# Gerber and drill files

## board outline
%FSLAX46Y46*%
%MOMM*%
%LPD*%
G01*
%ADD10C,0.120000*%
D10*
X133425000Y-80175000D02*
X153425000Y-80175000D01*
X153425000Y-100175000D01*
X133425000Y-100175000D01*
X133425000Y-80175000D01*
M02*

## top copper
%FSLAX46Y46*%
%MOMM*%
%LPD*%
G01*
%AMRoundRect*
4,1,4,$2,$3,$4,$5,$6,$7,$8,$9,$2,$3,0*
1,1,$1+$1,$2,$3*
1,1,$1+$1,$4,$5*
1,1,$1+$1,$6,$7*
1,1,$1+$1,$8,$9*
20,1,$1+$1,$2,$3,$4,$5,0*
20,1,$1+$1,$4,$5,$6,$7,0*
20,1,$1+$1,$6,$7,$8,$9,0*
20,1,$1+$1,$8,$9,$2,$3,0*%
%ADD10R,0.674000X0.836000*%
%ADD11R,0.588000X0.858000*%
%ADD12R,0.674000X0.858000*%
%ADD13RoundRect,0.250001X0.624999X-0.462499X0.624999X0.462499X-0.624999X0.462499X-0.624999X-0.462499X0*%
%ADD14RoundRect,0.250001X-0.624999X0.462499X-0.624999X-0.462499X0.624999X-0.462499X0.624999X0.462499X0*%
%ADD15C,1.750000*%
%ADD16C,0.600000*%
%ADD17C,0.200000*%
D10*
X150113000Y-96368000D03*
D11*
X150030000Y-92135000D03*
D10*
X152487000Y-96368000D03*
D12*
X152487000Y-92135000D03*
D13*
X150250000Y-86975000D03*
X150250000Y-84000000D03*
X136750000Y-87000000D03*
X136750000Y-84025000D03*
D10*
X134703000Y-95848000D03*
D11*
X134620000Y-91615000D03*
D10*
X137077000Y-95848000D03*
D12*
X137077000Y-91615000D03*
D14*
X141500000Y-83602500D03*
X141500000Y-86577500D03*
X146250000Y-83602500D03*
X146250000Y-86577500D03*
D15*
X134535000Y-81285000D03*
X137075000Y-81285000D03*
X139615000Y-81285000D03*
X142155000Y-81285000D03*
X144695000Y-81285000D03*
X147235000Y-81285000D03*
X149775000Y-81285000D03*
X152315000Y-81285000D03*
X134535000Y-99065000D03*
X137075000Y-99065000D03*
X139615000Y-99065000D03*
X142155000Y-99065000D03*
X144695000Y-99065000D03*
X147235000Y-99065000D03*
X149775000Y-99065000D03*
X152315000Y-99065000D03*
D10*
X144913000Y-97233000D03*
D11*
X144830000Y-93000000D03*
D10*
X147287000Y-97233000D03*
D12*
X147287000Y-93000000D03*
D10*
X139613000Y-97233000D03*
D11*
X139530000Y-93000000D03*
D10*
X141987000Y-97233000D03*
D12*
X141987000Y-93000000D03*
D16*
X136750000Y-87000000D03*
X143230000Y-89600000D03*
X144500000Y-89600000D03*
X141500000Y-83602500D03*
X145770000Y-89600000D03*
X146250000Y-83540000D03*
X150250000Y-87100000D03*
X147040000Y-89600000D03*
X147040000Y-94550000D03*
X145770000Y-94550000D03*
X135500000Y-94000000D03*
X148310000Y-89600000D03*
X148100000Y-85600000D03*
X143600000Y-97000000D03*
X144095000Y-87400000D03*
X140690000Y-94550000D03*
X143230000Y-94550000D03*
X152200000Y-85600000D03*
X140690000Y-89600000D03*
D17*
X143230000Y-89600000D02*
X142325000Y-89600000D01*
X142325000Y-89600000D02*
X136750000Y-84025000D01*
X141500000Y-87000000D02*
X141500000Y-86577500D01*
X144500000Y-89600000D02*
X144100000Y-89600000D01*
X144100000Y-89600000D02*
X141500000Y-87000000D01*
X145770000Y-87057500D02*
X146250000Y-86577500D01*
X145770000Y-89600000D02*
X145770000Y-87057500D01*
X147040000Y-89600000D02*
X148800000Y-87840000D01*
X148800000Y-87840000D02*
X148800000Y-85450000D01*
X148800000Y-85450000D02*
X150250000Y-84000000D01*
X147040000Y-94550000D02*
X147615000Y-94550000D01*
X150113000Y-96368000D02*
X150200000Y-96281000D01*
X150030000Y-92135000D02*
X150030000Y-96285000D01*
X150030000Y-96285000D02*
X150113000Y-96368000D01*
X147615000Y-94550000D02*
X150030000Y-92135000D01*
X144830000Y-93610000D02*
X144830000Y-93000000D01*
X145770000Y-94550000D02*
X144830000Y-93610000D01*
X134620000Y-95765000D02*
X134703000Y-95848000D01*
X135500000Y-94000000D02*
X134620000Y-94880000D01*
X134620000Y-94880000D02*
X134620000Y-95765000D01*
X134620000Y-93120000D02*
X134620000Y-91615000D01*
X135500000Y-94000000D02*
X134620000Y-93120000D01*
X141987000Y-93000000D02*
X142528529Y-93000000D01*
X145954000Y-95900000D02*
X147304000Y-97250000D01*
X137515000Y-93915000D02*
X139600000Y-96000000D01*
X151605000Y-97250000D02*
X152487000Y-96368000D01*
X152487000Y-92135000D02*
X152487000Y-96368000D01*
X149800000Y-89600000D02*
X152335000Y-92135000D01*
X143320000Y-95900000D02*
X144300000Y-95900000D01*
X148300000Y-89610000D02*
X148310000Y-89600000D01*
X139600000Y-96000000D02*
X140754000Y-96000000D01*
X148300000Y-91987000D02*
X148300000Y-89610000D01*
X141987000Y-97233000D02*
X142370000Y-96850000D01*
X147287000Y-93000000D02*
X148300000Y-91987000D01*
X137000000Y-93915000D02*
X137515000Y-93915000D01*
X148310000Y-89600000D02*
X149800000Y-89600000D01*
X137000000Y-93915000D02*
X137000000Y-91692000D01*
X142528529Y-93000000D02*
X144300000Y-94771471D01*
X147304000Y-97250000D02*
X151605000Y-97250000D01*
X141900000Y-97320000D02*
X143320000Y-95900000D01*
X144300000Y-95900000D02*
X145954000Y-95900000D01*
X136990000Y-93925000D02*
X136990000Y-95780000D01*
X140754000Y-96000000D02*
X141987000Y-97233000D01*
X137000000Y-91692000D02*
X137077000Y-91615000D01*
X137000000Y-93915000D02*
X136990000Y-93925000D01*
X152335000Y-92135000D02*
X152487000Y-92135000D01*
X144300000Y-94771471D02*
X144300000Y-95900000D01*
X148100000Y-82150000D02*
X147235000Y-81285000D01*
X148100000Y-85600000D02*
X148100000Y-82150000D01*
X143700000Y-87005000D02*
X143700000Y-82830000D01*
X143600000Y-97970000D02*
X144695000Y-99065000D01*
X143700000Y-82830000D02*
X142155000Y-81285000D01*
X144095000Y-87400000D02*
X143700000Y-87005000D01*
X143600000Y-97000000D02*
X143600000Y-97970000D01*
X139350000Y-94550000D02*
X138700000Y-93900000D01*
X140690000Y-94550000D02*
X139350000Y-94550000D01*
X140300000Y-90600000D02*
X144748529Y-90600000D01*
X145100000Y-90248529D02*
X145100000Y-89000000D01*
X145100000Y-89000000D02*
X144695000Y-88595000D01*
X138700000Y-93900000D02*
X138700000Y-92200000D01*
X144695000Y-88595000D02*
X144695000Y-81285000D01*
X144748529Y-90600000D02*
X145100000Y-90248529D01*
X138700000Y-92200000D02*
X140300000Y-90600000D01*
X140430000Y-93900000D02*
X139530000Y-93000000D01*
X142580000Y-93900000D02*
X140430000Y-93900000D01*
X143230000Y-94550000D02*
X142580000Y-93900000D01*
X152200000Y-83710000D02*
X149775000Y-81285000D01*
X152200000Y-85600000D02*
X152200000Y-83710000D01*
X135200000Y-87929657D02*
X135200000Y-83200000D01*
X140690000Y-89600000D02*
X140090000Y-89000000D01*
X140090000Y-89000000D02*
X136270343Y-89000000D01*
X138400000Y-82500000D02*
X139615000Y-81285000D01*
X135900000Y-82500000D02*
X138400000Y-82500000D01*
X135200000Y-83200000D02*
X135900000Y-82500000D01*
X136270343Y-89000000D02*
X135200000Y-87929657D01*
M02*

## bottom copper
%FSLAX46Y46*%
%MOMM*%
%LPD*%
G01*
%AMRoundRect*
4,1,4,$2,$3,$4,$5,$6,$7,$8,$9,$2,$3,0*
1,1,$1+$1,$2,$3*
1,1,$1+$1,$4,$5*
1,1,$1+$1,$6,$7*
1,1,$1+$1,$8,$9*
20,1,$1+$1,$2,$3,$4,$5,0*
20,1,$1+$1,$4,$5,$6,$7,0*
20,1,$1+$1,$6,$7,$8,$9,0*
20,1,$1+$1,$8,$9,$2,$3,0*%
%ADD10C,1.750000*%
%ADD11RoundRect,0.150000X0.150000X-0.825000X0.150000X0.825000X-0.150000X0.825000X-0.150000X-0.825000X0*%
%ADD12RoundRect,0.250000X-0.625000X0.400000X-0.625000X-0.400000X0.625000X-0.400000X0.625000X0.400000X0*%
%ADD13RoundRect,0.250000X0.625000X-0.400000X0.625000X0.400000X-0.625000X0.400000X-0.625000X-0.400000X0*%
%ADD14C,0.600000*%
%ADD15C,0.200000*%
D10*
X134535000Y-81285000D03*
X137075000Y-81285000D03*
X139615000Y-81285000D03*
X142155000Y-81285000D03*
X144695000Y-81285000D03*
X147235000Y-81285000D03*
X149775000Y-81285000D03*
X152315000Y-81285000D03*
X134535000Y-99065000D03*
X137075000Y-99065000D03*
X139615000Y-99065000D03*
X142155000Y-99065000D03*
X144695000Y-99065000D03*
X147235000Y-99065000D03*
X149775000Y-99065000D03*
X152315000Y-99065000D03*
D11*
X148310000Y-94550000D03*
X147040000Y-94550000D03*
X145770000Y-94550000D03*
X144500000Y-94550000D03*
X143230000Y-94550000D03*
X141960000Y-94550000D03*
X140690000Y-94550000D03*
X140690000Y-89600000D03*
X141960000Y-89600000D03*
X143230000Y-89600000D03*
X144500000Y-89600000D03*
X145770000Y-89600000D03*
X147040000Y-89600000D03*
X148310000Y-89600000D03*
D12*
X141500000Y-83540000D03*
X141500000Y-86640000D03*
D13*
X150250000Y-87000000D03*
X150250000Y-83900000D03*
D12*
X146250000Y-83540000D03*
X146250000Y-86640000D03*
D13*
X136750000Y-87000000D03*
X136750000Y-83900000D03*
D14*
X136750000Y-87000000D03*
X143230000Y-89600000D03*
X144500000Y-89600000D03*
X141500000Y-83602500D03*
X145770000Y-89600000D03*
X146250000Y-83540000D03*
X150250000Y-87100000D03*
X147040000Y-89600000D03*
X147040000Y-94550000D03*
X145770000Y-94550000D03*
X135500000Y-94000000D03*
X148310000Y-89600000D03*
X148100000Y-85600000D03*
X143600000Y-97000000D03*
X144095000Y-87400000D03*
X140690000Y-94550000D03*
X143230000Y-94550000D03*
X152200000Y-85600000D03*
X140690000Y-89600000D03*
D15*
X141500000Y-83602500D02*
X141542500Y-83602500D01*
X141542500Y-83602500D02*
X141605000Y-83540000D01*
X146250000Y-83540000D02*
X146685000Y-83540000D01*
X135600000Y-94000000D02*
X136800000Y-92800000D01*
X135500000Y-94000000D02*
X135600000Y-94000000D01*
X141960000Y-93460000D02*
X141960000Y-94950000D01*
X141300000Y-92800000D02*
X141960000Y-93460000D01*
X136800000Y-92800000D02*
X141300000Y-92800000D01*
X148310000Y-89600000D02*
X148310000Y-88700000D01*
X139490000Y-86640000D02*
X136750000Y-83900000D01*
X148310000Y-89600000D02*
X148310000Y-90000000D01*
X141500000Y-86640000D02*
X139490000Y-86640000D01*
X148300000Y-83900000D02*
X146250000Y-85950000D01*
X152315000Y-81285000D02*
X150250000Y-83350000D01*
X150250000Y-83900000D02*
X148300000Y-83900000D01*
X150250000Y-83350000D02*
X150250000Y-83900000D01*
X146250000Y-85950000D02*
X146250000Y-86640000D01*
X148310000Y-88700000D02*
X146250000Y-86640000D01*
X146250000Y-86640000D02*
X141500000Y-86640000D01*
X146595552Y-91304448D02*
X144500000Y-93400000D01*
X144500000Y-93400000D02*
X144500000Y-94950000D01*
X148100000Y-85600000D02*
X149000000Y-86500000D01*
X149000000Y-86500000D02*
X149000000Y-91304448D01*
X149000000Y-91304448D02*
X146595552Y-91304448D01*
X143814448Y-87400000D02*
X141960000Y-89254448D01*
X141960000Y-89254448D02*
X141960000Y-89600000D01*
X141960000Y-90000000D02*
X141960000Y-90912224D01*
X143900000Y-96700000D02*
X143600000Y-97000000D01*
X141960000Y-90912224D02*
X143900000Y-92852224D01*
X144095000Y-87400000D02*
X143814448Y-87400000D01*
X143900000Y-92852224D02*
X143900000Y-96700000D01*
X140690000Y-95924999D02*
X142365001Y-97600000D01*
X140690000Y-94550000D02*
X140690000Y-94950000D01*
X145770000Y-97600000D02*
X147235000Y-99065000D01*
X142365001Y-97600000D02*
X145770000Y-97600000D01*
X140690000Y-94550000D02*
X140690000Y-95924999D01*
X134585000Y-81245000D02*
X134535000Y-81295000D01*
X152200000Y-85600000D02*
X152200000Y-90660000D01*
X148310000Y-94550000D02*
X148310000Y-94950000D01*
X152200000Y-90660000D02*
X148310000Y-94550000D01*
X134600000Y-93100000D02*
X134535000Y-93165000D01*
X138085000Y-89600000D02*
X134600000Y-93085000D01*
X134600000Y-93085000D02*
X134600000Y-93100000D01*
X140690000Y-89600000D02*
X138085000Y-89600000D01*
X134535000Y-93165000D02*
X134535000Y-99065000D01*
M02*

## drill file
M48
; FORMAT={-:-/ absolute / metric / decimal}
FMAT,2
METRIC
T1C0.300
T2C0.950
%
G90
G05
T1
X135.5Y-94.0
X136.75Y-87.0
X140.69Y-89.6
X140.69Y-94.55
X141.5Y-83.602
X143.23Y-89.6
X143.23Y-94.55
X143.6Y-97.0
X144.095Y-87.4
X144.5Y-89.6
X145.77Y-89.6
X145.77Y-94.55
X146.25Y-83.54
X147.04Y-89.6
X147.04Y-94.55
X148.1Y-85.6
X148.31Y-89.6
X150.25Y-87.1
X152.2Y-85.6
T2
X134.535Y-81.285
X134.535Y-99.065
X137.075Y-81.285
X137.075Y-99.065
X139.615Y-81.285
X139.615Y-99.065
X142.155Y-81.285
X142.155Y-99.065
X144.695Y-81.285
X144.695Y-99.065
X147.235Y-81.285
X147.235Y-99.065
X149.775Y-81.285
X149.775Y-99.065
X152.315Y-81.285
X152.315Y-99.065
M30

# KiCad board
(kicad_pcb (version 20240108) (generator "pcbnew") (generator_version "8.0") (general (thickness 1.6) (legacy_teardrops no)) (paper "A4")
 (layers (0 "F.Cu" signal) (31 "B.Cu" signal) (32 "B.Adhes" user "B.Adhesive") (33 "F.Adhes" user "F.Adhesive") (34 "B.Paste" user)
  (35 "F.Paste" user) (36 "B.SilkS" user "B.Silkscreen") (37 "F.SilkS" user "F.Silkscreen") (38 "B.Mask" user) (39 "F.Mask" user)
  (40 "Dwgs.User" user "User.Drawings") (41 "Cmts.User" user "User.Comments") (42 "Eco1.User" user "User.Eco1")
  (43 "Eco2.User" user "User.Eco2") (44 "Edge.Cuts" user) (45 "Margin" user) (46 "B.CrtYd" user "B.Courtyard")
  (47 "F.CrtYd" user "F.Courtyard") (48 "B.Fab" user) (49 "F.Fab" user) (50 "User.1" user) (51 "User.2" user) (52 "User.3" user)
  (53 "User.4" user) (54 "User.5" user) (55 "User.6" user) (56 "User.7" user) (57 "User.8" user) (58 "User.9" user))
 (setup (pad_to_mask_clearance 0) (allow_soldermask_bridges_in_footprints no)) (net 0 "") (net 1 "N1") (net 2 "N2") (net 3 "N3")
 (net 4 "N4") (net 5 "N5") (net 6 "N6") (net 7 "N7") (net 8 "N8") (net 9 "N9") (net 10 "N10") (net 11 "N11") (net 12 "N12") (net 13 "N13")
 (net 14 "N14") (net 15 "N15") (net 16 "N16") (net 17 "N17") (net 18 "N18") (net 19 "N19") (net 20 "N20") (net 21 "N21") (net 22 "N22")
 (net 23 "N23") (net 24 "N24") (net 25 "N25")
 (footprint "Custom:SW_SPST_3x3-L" (layer "F.Cu") (at 151.3 94.5 90)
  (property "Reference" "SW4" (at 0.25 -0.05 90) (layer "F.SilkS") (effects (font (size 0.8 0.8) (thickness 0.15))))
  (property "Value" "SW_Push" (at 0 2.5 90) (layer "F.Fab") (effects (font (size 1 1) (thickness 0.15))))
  (pad "1" smd rect (at -1.868 -1.187 90) (size 0.836 0.674) (layers "F.Cu" "F.Paste" "F.Mask") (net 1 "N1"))
  (pad "1" smd rect (at 2.365 -1.27 90) (size 0.858 0.588) (layers "F.Cu" "F.Paste" "F.Mask") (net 1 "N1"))
  (pad "2" smd rect (at -1.868 1.187 90) (size 0.836 0.674) (layers "F.Cu" "F.Paste" "F.Mask") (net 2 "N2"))
  (pad "2" smd rect (at 2.365 1.187 90) (size 0.858 0.674) (layers "F.Cu" "F.Paste" "F.Mask") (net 2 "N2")))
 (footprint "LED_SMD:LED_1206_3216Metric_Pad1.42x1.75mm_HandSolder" (layer "F.Cu") (at 150.25 85.4875 90)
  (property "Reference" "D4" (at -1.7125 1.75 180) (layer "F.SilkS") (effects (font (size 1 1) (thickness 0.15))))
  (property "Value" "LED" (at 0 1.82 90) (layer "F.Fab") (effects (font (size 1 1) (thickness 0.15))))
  (pad "1" smd roundrect (at -1.4875 0 90) (size 1.425 1.75) (layers "F.Cu" "F.Paste" "F.Mask") (roundrect_rratio 0.175439) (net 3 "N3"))
  (pad "2" smd roundrect (at 1.4875 0 90) (size 1.425 1.75) (layers "F.Cu" "F.Paste" "F.Mask") (roundrect_rratio 0.175439) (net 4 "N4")))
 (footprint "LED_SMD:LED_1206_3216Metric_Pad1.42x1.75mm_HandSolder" (layer "F.Cu") (at 136.75 85.5125 90)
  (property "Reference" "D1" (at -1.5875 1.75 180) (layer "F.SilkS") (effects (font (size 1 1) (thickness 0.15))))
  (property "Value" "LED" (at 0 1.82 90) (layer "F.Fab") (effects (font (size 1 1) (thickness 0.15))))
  (pad "1" smd roundrect (at -1.4875 0 90) (size 1.425 1.75) (layers "F.Cu" "F.Paste" "F.Mask") (roundrect_rratio 0.175439) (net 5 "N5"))
  (pad "2" smd roundrect (at 1.4875 0 90) (size 1.425 1.75) (layers "F.Cu" "F.Paste" "F.Mask") (roundrect_rratio 0.175439) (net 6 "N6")))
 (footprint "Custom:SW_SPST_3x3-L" (layer "F.Cu") (at 135.89 93.98 90)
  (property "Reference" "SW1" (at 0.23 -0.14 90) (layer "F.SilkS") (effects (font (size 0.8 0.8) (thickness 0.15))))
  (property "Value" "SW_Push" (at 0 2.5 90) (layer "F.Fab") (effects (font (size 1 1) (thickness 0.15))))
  (pad "1" smd rect (at -1.868 -1.187 90) (size 0.836 0.674) (layers "F.Cu" "F.Paste" "F.Mask") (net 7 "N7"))
  (pad "1" smd rect (at 2.365 -1.27 90) (size 0.858 0.588) (layers "F.Cu" "F.Paste" "F.Mask") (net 7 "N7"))
  (pad "2" smd rect (at -1.868 1.187 90) (size 0.836 0.674) (layers "F.Cu" "F.Paste" "F.Mask") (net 2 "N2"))
  (pad "2" smd rect (at 2.365 1.187 90) (size 0.858 0.674) (layers "F.Cu" "F.Paste" "F.Mask") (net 2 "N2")))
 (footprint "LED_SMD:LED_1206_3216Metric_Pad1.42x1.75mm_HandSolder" (layer "F.Cu") (at 141.5 85.09 -90)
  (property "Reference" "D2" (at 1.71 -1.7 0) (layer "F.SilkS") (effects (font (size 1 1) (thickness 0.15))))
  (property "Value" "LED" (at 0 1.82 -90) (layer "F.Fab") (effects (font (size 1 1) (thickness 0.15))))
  (pad "1" smd roundrect (at -1.4875 0 270) (size 1.425 1.75) (layers "F.Cu" "F.Paste" "F.Mask") (roundrect_rratio 0.175439) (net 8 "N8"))
  (pad "2" smd roundrect (at 1.4875 0 270) (size 1.425 1.75) (layers "F.Cu" "F.Paste" "F.Mask") (roundrect_rratio 0.175439) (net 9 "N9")))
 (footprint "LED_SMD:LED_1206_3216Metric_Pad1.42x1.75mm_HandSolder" (layer "F.Cu") (at 146.25 85.09 -90)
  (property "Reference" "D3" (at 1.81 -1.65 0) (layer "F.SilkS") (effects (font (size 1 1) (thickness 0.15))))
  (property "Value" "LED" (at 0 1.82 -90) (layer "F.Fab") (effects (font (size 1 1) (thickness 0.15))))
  (pad "1" smd roundrect (at -1.4875 0 270) (size 1.425 1.75) (layers "F.Cu" "F.Paste" "F.Mask") (roundrect_rratio 0.175439) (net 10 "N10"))
  (pad "2" smd roundrect (at 1.4875 0 270) (size 1.425 1.75) (layers "F.Cu" "F.Paste" "F.Mask") (roundrect_rratio 0.175439) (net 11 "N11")))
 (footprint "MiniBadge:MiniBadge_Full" (layer "F.Cu") (at 133.265 80.015)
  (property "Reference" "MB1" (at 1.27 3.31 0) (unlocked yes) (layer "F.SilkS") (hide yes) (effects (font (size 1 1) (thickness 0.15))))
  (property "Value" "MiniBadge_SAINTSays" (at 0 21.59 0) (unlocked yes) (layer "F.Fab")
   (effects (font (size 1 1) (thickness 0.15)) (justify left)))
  (fp_rect (start 20.16 20.16) (end 0.16 0.16) (stroke (width 0.12) (type solid)) (fill none) (layer "Edge.Cuts"))
  (pad "1" thru_hole circle (at 1.27 1.27) (size 1.75 1.75) (drill 0.95) (layers "*.Cu" "*.Mask") (remove_unused_layers no) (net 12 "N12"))
  (pad "2" thru_hole circle (at 3.81 1.27) (size 1.75 1.75) (drill 0.95) (layers "*.Cu" "*.Mask") (remove_unused_layers no) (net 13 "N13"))
  (pad "3" thru_hole circle (at 6.35 1.27 90) (size 1.75 1.75) (drill 0.95) (layers "*.Cu" "*.Mask") (remove_unused_layers no)
   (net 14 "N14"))
  (pad "4" thru_hole circle (at 8.89 1.27) (size 1.75 1.75) (drill 0.95) (layers "*.Cu" "*.Mask") (remove_unused_layers no) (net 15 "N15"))
  (pad "5" thru_hole circle (at 11.43 1.27) (size 1.75 1.75) (drill 0.95) (layers "*.Cu" "*.Mask") (remove_unused_layers no) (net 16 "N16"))
  (pad "6" thru_hole circle (at 13.97 1.27) (size 1.75 1.75) (drill 0.95) (layers "*.Cu" "*.Mask") (remove_unused_layers no) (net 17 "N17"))
  (pad "7" thru_hole circle (at 16.51 1.27) (size 1.75 1.75) (drill 0.95) (layers "*.Cu" "*.Mask") (remove_unused_layers no) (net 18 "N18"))
  (pad "8" thru_hole circle (at 19.05 1.27) (size 1.75 1.75) (drill 0.95) (layers "*.Cu" "*.Mask") (remove_unused_layers no) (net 2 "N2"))
  (pad "9" thru_hole circle (at 1.27 19.05) (size 1.75 1.75) (drill 0.95) (layers "*.Cu" "*.Mask") (remove_unused_layers no) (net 14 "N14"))
  (pad "10" thru_hole circle (at 3.81 19.05) (size 1.75 1.75) (drill 0.95) (layers "*.Cu" "*.Mask") (remove_unused_layers no) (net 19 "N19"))
  (pad "11" thru_hole circle (at 6.35 19.05) (size 1.75 1.75) (drill 0.95) (layers "*.Cu" "*.Mask") (remove_unused_layers no) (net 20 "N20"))
  (pad "12" thru_hole circle (at 8.89 19.05) (size 1.75 1.75) (drill 0.95) (layers "*.Cu" "*.Mask") (remove_unused_layers no) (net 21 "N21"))
  (pad "13" thru_hole circle (at 11.43 19.05) (size 1.75 1.75) (drill 0.95) (layers "*.Cu" "*.Mask") (remove_unused_layers no)
   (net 15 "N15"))
  (pad "14" thru_hole circle (at 13.97 19.05) (size 1.75 1.75) (drill 0.95) (layers "*.Cu" "*.Mask") (remove_unused_layers no)
   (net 16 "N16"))
  (pad "15" thru_hole circle (at 16.51 19.05) (size 1.75 1.75) (drill 0.95) (layers "*.Cu" "*.Mask") (remove_unused_layers no)
   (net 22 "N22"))
  (pad "16" thru_hole circle (at 19.05 19.05) (size 1.75 1.75) (drill 0.95) (layers "*.Cu" "*.Mask") (remove_unused_layers no)
   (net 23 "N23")))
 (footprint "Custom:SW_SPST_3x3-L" (layer "F.Cu") (at 146.1 95.365 90)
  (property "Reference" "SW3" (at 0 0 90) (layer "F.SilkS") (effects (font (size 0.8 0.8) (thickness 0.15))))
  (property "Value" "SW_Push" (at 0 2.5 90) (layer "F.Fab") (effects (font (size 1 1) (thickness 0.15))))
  (pad "1" smd rect (at -1.868 -1.187 90) (size 0.836 0.674) (layers "F.Cu" "F.Paste" "F.Mask") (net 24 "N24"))
  (pad "1" smd rect (at 2.365 -1.27 90) (size 0.858 0.588) (layers "F.Cu" "F.Paste" "F.Mask") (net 24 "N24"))
  (pad "2" smd rect (at -1.868 1.187 90) (size 0.836 0.674) (layers "F.Cu" "F.Paste" "F.Mask") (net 2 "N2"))
  (pad "2" smd rect (at 2.365 1.187 90) (size 0.858 0.674) (layers "F.Cu" "F.Paste" "F.Mask") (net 2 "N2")))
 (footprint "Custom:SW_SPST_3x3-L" (layer "F.Cu") (at 140.8 95.365 90)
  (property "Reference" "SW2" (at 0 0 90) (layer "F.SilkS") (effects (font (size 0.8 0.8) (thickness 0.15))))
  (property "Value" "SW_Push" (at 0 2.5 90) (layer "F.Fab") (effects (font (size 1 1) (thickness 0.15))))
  (pad "1" smd rect (at -1.868 -1.187 90) (size 0.836 0.674) (layers "F.Cu" "F.Paste" "F.Mask") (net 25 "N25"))
  (pad "1" smd rect (at 2.365 -1.27 90) (size 0.858 0.588) (layers "F.Cu" "F.Paste" "F.Mask") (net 25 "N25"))
  (pad "2" smd rect (at -1.868 1.187 90) (size 0.836 0.674) (layers "F.Cu" "F.Paste" "F.Mask") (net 2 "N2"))
  (pad "2" smd rect (at 2.365 1.187 90) (size 0.858 0.674) (layers "F.Cu" "F.Paste" "F.Mask") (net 2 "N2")))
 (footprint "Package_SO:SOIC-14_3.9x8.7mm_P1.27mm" (layer "B.Cu") (at 144.5 92.075 90)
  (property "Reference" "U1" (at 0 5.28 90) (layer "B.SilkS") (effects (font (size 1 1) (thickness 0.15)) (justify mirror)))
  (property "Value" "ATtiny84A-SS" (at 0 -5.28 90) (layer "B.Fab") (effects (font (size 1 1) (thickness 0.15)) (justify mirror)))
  (pad "1" smd roundrect (at -2.475 3.81 90) (size 1.95 0.6) (layers "B.Cu" "B.Paste" "B.Mask") (roundrect_rratio 0.25) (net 18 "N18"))
  (pad "2" smd roundrect (at -2.475 2.54 90) (size 1.95 0.6) (layers "B.Cu" "B.Paste" "B.Mask") (roundrect_rratio 0.25) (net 1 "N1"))
  (pad "3" smd roundrect (at -2.475 1.27 90) (size 1.95 0.6) (layers "B.Cu" "B.Paste" "B.Mask") (roundrect_rratio 0.25) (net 24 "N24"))
  (pad "4" smd roundrect (at -2.475 0 90) (size 1.95 0.6) (layers "B.Cu" "B.Paste" "B.Mask") (roundrect_rratio 0.25) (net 17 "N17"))
  (pad "5" smd roundrect (at -2.475 -1.27 90) (size 1.95 0.6) (layers "B.Cu" "B.Paste" "B.Mask") (roundrect_rratio 0.25) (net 25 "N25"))
  (pad "6" smd roundrect (at -2.475 -2.54 90) (size 1.95 0.6) (layers "B.Cu" "B.Paste" "B.Mask") (roundrect_rratio 0.25) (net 7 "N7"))
  (pad "7" smd roundrect (at -2.475 -3.81 90) (size 1.95 0.6) (layers "B.Cu" "B.Paste" "B.Mask") (roundrect_rratio 0.25) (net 16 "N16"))
  (pad "8" smd roundrect (at 2.475 -3.81 90) (size 1.95 0.6) (layers "B.Cu" "B.Paste" "B.Mask") (roundrect_rratio 0.25) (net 14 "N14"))
  (pad "9" smd roundrect (at 2.475 -2.54 90) (size 1.95 0.6) (layers "B.Cu" "B.Paste" "B.Mask") (roundrect_rratio 0.25) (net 15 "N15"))
  (pad "10" smd roundrect (at 2.475 -1.27 90) (size 1.95 0.6) (layers "B.Cu" "B.Paste" "B.Mask") (roundrect_rratio 0.25) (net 6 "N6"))
  (pad "11" smd roundrect (at 2.475 0 90) (size 1.95 0.6) (layers "B.Cu" "B.Paste" "B.Mask") (roundrect_rratio 0.25) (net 9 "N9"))
  (pad "12" smd roundrect (at 2.475 1.27 90) (size 1.95 0.6) (layers "B.Cu" "B.Paste" "B.Mask") (roundrect_rratio 0.25) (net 11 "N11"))
  (pad "13" smd roundrect (at 2.475 2.54 90) (size 1.95 0.6) (layers "B.Cu" "B.Paste" "B.Mask") (roundrect_rratio 0.25) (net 4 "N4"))
  (pad "14" smd roundrect (at 2.475 3.81 90) (size 1.95 0.6) (layers "B.Cu" "B.Paste" "B.Mask") (roundrect_rratio 0.25) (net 2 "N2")))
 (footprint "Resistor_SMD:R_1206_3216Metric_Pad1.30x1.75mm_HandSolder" (layer "B.Cu") (at 141.5 85.09 -90)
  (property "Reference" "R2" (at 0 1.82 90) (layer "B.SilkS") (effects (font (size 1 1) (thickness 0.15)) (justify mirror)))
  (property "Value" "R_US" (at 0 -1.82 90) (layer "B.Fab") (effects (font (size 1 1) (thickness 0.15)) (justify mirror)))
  (pad "1" smd roundrect (at -1.55 0 270) (size 1.3 1.75) (layers "B.Cu" "B.Paste" "B.Mask") (roundrect_rratio 0.192308) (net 8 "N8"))
  (pad "2" smd roundrect (at 1.55 0 270) (size 1.3 1.75) (layers "B.Cu" "B.Paste" "B.Mask") (roundrect_rratio 0.192308) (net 2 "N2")))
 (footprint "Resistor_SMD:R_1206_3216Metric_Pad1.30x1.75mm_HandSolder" (layer "B.Cu") (at 150.25 85.45 90)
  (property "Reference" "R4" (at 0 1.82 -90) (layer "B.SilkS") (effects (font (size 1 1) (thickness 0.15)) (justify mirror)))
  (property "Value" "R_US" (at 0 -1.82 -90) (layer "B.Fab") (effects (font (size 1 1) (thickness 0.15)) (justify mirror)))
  (pad "1" smd roundrect (at -1.55 0 90) (size 1.3 1.75) (layers "B.Cu" "B.Paste" "B.Mask") (roundrect_rratio 0.192308) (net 3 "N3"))
  (pad "2" smd roundrect (at 1.55 0 90) (size 1.3 1.75) (layers "B.Cu" "B.Paste" "B.Mask") (roundrect_rratio 0.192308) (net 2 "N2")))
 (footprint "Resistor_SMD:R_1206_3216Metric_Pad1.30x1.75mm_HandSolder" (layer "B.Cu") (at 146.25 85.09 -90)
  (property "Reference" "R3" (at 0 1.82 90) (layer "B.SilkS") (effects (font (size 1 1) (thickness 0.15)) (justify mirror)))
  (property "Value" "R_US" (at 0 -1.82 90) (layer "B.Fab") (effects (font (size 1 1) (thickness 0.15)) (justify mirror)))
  (pad "1" smd roundrect (at -1.55 0 270) (size 1.3 1.75) (layers "B.Cu" "B.Paste" "B.Mask") (roundrect_rratio 0.192308) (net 10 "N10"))
  (pad "2" smd roundrect (at 1.55 0 270) (size 1.3 1.75) (layers "B.Cu" "B.Paste" "B.Mask") (roundrect_rratio 0.192308) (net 2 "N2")))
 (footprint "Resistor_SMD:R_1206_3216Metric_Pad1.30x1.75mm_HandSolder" (layer "B.Cu") (at 136.75 85.45 90)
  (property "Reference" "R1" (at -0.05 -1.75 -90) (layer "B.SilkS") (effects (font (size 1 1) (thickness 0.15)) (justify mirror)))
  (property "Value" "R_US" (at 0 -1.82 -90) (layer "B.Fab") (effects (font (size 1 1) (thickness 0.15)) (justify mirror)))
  (pad "1" smd roundrect (at -1.55 0 90) (size 1.3 1.75) (layers "B.Cu" "B.Paste" "B.Mask") (roundrect_rratio 0.192308) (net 5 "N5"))
  (pad "2" smd roundrect (at 1.55 0 90) (size 1.3 1.75) (layers "B.Cu" "B.Paste" "B.Mask") (roundrect_rratio 0.192308) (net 2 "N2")))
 (via (at 136.75 87) (size 0.6) (drill 0.3) (layers "F.Cu" "B.Cu") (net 5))
 (segment (start 143.23 89.6) (end 142.325 89.6) (width 0.2) (layer "F.Cu") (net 6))
 (segment (start 142.325 89.6) (end 136.75 84.025) (width 0.2) (layer "F.Cu") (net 6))
 (via (at 143.23 89.6) (size 0.6) (drill 0.3) (layers "F.Cu" "B.Cu") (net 6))
 (segment (start 141.5 87) (end 141.5 86.5775) (width 0.2) (layer "F.Cu") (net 9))
 (segment (start 144.5 89.6) (end 144.1 89.6) (width 0.2) (layer "F.Cu") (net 9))
 (segment (start 144.1 89.6) (end 141.5 87) (width 0.2) (layer "F.Cu") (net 9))
 (via (at 144.5 89.6) (size 0.6) (drill 0.3) (layers "F.Cu" "B.Cu") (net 9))
 (via (at 141.5 83.6025) (size 0.6) (drill 0.3) (layers "F.Cu" "B.Cu") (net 8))
 (segment (start 141.5 83.6025) (end 141.5425 83.6025) (width 0.2) (layer "B.Cu") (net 8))
 (segment (start 141.5425 83.6025) (end 141.605 83.54) (width 0.2) (layer "B.Cu") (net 8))
 (segment (start 145.77 87.0575) (end 146.25 86.5775) (width 0.2) (layer "F.Cu") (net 11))
 (segment (start 145.77 89.6) (end 145.77 87.0575) (width 0.2) (layer "F.Cu") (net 11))
 (via (at 145.77 89.6) (size 0.6) (drill 0.3) (layers "F.Cu" "B.Cu") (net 11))
 (via (at 146.25 83.54) (size 0.6) (drill 0.3) (layers "F.Cu" "B.Cu") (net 10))
 (segment (start 146.25 83.54) (end 146.685 83.54) (width 0.2) (layer "B.Cu") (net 10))
 (via (at 150.25 87.1) (size 0.6) (drill 0.3) (layers "F.Cu" "B.Cu") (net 3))
 (segment (start 147.04 89.6) (end 148.8 87.84) (width 0.2) (layer "F.Cu") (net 4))
 (segment (start 148.8 87.84) (end 148.8 85.45) (width 0.2) (layer "F.Cu") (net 4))
 (segment (start 148.8 85.45) (end 150.25 84) (width 0.2) (layer "F.Cu") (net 4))
 (via (at 147.04 89.6) (size 0.6) (drill 0.3) (layers "F.Cu" "B.Cu") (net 4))
 (segment (start 147.04 94.55) (end 147.615 94.55) (width 0.2) (layer "F.Cu") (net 1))
 (segment (start 150.113 96.368) (end 150.2 96.281) (width 0.2) (layer "F.Cu") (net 1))
 (segment (start 150.03 92.135) (end 150.03 96.285) (width 0.2) (layer "F.Cu") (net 1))
 (segment (start 150.03 96.285) (end 150.113 96.368) (width 0.2) (layer "F.Cu") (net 1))
 (segment (start 147.615 94.55) (end 150.03 92.135) (width 0.2) (layer "F.Cu") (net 1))
 (via (at 147.04 94.55) (size 0.6) (drill 0.3) (layers "F.Cu" "B.Cu") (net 1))
 (segment (start 144.83 93.61) (end 144.83 93) (width 0.2) (layer "F.Cu") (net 24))
 (segment (start 145.77 94.55) (end 144.83 93.61) (width 0.2) (layer "F.Cu") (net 24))
 (via (at 145.77 94.55) (size 0.6) (drill 0.3) (layers "F.Cu" "B.Cu") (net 24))
 (segment (start 134.62 95.765) (end 134.703 95.848) (width 0.2) (layer "F.Cu") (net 7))
 (segment (start 135.5 94) (end 134.62 94.88) (width 0.2) (layer "F.Cu") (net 7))
 (segment (start 134.62 94.88) (end 134.62 95.765) (width 0.2) (layer "F.Cu") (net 7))
 (segment (start 134.62 93.12) (end 134.62 91.615) (width 0.2) (layer "F.Cu") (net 7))
 (segment (start 135.5 94) (end 134.62 93.12) (width 0.2) (layer "F.Cu") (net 7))
 (via (at 135.5 94) (size 0.6) (drill 0.3) (layers "F.Cu" "B.Cu") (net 7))
 (segment (start 135.6 94) (end 136.8 92.8) (width 0.2) (layer "B.Cu") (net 7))
 (segment (start 135.5 94) (end 135.6 94) (width 0.2) (layer "B.Cu") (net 7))
 (segment (start 141.96 93.46) (end 141.96 94.95) (width 0.2) (layer "B.Cu") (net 7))
 (segment (start 141.3 92.8) (end 141.96 93.46) (width 0.2) (layer "B.Cu") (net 7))
 (segment (start 136.8 92.8) (end 141.3 92.8) (width 0.2) (layer "B.Cu") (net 7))
 (segment (start 141.987 93) (end 142.528529 93) (width 0.2) (layer "F.Cu") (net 2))
 (segment (start 145.954 95.9) (end 147.304 97.25) (width 0.2) (layer "F.Cu") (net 2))
 (segment (start 137.515 93.915) (end 139.6 96) (width 0.2) (layer "F.Cu") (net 2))
 (segment (start 151.605 97.25) (end 152.487 96.368) (width 0.2) (layer "F.Cu") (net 2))
 (segment (start 152.487 92.135) (end 152.487 96.368) (width 0.2) (layer "F.Cu") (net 2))
 (segment (start 149.8 89.6) (end 152.335 92.135) (width 0.2) (layer "F.Cu") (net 2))
 (segment (start 143.32 95.9) (end 144.3 95.9) (width 0.2) (layer "F.Cu") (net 2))
 (segment (start 148.3 89.61) (end 148.31 89.6) (width 0.2) (layer "F.Cu") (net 2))
 (segment (start 139.6 96) (end 140.754 96) (width 0.2) (layer "F.Cu") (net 2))
 (segment (start 148.3 91.987) (end 148.3 89.61) (width 0.2) (layer "F.Cu") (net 2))
 (segment (start 141.987 97.233) (end 142.37 96.85) (width 0.2) (layer "F.Cu") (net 2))
 (segment (start 147.287 93) (end 148.3 91.987) (width 0.2) (layer "F.Cu") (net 2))
 (segment (start 137 93.915) (end 137.515 93.915) (width 0.2) (layer "F.Cu") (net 2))
 (segment (start 148.31 89.6) (end 149.8 89.6) (width 0.2) (layer "F.Cu") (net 2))
 (segment (start 137 93.915) (end 137 91.692) (width 0.2) (layer "F.Cu") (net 2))
 (segment (start 142.528529 93) (end 144.3 94.771471) (width 0.2) (layer "F.Cu") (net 2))
 (segment (start 147.304 97.25) (end 151.605 97.25) (width 0.2) (layer "F.Cu") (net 2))
 (segment (start 141.9 97.32) (end 143.32 95.9) (width 0.2) (layer "F.Cu") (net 2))
 (segment (start 144.3 95.9) (end 145.954 95.9) (width 0.2) (layer "F.Cu") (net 2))
 (segment (start 136.99 93.925) (end 136.99 95.78) (width 0.2) (layer "F.Cu") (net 2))
 (segment (start 140.754 96) (end 141.987 97.233) (width 0.2) (layer "F.Cu") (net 2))
 (segment (start 137 91.692) (end 137.077 91.615) (width 0.2) (layer "F.Cu") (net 2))
 (segment (start 137 93.915) (end 136.99 93.925) (width 0.2) (layer "F.Cu") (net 2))
 (segment (start 152.335 92.135) (end 152.487 92.135) (width 0.2) (layer "F.Cu") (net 2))
 (segment (start 144.3 94.771471) (end 144.3 95.9) (width 0.2) (layer "F.Cu") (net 2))
 (via (at 148.31 89.6) (size 0.6) (drill 0.3) (layers "F.Cu" "B.Cu") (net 2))
 (segment (start 148.31 89.6) (end 148.31 88.7) (width 0.2) (layer "B.Cu") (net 2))
 (segment (start 139.49 86.64) (end 136.75 83.9) (width 0.2) (layer "B.Cu") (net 2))
 (segment (start 148.31 89.6) (end 148.31 90) (width 0.2) (layer "B.Cu") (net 2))
 (segment (start 141.5 86.64) (end 139.49 86.64) (width 0.2) (layer "B.Cu") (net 2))
 (segment (start 148.3 83.9) (end 146.25 85.95) (width 0.2) (layer "B.Cu") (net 2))
 (segment (start 152.315 81.285) (end 150.25 83.35) (width 0.2) (layer "B.Cu") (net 2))
 (segment (start 150.25 83.9) (end 148.3 83.9) (width 0.2) (layer "B.Cu") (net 2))
 (segment (start 150.25 83.35) (end 150.25 83.9) (width 0.2) (layer "B.Cu") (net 2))
 (segment (start 146.25 85.95) (end 146.25 86.64) (width 0.2) (layer "B.Cu") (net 2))
 (segment (start 148.31 88.7) (end 146.25 86.64) (width 0.2) (layer "B.Cu") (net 2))
 (segment (start 146.25 86.64) (end 141.5 86.64) (width 0.2) (layer "B.Cu") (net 2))
 (segment (start 148.1 82.15) (end 147.235 81.285) (width 0.2) (layer "F.Cu") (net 17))
 (segment (start 148.1 85.6) (end 148.1 82.15) (width 0.2) (layer "F.Cu") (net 17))
 (via (at 148.1 85.6) (size 0.6) (drill 0.3) (layers "F.Cu" "B.Cu") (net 17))
 (segment (start 146.595552 91.304448) (end 144.5 93.4) (width 0.2) (layer "B.Cu") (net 17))
 (segment (start 144.5 93.4) (end 144.5 94.95) (width 0.2) (layer "B.Cu") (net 17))
 (segment (start 148.1 85.6) (end 149 86.5) (width 0.2) (layer "B.Cu") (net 17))
 (segment (start 149 86.5) (end 149 91.304448) (width 0.2) (layer "B.Cu") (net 17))
 (segment (start 149 91.304448) (end 146.595552 91.304448) (width 0.2) (layer "B.Cu") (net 17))
 (segment (start 143.7 87.005) (end 143.7 82.83) (width 0.2) (layer "F.Cu") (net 15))
 (segment (start 143.6 97.97) (end 144.695 99.065) (width 0.2) (layer "F.Cu") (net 15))
 (segment (start 143.7 82.83) (end 142.155 81.285) (width 0.2) (layer "F.Cu") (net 15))
 (segment (start 144.095 87.4) (end 143.7 87.005) (width 0.2) (layer "F.Cu") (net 15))
 (segment (start 143.6 97) (end 143.6 97.97) (width 0.2) (layer "F.Cu") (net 15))
 (via (at 143.6 97) (size 0.6) (drill 0.3) (layers "F.Cu" "B.Cu") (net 15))
 (via (at 144.095 87.4) (size 0.6) (drill 0.3) (layers "F.Cu" "B.Cu") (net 15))
 (segment (start 143.814448 87.4) (end 141.96 89.254448) (width 0.2) (layer "B.Cu") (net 15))
 (segment (start 141.96 89.254448) (end 141.96 89.6) (width 0.2) (layer "B.Cu") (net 15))
 (segment (start 141.96 90) (end 141.96 90.912224) (width 0.2) (layer "B.Cu") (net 15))
 (segment (start 143.9 96.7) (end 143.6 97) (width 0.2) (layer "B.Cu") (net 15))
 (segment (start 141.96 90.912224) (end 143.9 92.852224) (width 0.2) (layer "B.Cu") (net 15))
 (segment (start 144.095 87.4) (end 143.814448 87.4) (width 0.2) (layer "B.Cu") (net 15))
 (segment (start 143.9 92.852224) (end 143.9 96.7) (width 0.2) (layer "B.Cu") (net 15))
 (segment (start 139.35 94.55) (end 138.7 93.9) (width 0.2) (layer "F.Cu") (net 16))
 (segment (start 140.69 94.55) (end 139.35 94.55) (width 0.2) (layer "F.Cu") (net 16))
 (segment (start 140.3 90.6) (end 144.748529 90.6) (width 0.2) (layer "F.Cu") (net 16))
 (segment (start 145.1 90.248529) (end 145.1 89) (width 0.2) (layer "F.Cu") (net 16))
 (segment (start 145.1 89) (end 144.695 88.595) (width 0.2) (layer "F.Cu") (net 16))
 (segment (start 138.7 93.9) (end 138.7 92.2) (width 0.2) (layer "F.Cu") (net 16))
 (segment (start 144.695 88.595) (end 144.695 81.285) (width 0.2) (layer "F.Cu") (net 16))
 (segment (start 144.748529 90.6) (end 145.1 90.248529) (width 0.2) (layer "F.Cu") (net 16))
 (segment (start 138.7 92.2) (end 140.3 90.6) (width 0.2) (layer "F.Cu") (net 16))
 (via (at 140.69 94.55) (size 0.6) (drill 0.3) (layers "F.Cu" "B.Cu") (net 16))
 (segment (start 140.69 95.924999) (end 142.365001 97.6) (width 0.2) (layer "B.Cu") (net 16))
 (segment (start 140.69 94.55) (end 140.69 94.95) (width 0.2) (layer "B.Cu") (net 16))
 (segment (start 145.77 97.6) (end 147.235 99.065) (width 0.2) (layer "B.Cu") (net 16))
 (segment (start 142.365001 97.6) (end 145.77 97.6) (width 0.2) (layer "B.Cu") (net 16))
 (segment (start 140.69 94.55) (end 140.69 95.924999) (width 0.2) (layer "B.Cu") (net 16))
 (segment (start 140.43 93.9) (end 139.53 93) (width 0.2) (layer "F.Cu") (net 25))
 (segment (start 142.58 93.9) (end 140.43 93.9) (width 0.2) (layer "F.Cu") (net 25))
 (segment (start 143.23 94.55) (end 142.58 93.9) (width 0.2) (layer "F.Cu") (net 25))
 (via (at 143.23 94.55) (size 0.6) (drill 0.3) (layers "F.Cu" "B.Cu") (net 25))
 (segment (start 134.585 81.245) (end 134.535 81.295) (width 0.2) (layer "B.Cu") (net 12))
 (segment (start 152.2 83.71) (end 149.775 81.285) (width 0.2) (layer "F.Cu") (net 18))
 (segment (start 152.2 85.6) (end 152.2 83.71) (width 0.2) (layer "F.Cu") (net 18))
 (via (at 152.2 85.6) (size 0.6) (drill 0.3) (layers "F.Cu" "B.Cu") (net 18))
 (segment (start 152.2 85.6) (end 152.2 90.66) (width 0.2) (layer "B.Cu") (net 18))
 (segment (start 148.31 94.55) (end 148.31 94.95) (width 0.2) (layer "B.Cu") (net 18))
 (segment (start 152.2 90.66) (end 148.31 94.55) (width 0.2) (layer "B.Cu") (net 18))
 (segment (start 135.2 87.929657) (end 135.2 83.2) (width 0.2) (layer "F.Cu") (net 14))
 (segment (start 140.69 89.6) (end 140.09 89) (width 0.2) (layer "F.Cu") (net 14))
 (segment (start 140.09 89) (end 136.270343 89) (width 0.2) (layer "F.Cu") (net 14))
 (segment (start 138.4 82.5) (end 139.615 81.285) (width 0.2) (layer "F.Cu") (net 14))
 (segment (start 135.9 82.5) (end 138.4 82.5) (width 0.2) (layer "F.Cu") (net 14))
 (segment (start 135.2 83.2) (end 135.9 82.5) (width 0.2) (layer "F.Cu") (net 14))
 (segment (start 136.270343 89) (end 135.2 87.929657) (width 0.2) (layer "F.Cu") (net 14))
 (via (at 140.69 89.6) (size 0.6) (drill 0.3) (layers "F.Cu" "B.Cu") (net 14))
 (segment (start 134.6 93.1) (end 134.535 93.165) (width 0.2) (layer "B.Cu") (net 14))
 (segment (start 138.085 89.6) (end 134.6 93.085) (width 0.2) (layer "B.Cu") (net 14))
 (segment (start 134.6 93.085) (end 134.6 93.1) (width 0.2) (layer "B.Cu") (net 14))
 (segment (start 140.69 89.6) (end 138.085 89.6) (width 0.2) (layer "B.Cu") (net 14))
 (segment (start 134.535 93.165) (end 134.535 99.065) (width 0.2) (layer "B.Cu") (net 14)))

